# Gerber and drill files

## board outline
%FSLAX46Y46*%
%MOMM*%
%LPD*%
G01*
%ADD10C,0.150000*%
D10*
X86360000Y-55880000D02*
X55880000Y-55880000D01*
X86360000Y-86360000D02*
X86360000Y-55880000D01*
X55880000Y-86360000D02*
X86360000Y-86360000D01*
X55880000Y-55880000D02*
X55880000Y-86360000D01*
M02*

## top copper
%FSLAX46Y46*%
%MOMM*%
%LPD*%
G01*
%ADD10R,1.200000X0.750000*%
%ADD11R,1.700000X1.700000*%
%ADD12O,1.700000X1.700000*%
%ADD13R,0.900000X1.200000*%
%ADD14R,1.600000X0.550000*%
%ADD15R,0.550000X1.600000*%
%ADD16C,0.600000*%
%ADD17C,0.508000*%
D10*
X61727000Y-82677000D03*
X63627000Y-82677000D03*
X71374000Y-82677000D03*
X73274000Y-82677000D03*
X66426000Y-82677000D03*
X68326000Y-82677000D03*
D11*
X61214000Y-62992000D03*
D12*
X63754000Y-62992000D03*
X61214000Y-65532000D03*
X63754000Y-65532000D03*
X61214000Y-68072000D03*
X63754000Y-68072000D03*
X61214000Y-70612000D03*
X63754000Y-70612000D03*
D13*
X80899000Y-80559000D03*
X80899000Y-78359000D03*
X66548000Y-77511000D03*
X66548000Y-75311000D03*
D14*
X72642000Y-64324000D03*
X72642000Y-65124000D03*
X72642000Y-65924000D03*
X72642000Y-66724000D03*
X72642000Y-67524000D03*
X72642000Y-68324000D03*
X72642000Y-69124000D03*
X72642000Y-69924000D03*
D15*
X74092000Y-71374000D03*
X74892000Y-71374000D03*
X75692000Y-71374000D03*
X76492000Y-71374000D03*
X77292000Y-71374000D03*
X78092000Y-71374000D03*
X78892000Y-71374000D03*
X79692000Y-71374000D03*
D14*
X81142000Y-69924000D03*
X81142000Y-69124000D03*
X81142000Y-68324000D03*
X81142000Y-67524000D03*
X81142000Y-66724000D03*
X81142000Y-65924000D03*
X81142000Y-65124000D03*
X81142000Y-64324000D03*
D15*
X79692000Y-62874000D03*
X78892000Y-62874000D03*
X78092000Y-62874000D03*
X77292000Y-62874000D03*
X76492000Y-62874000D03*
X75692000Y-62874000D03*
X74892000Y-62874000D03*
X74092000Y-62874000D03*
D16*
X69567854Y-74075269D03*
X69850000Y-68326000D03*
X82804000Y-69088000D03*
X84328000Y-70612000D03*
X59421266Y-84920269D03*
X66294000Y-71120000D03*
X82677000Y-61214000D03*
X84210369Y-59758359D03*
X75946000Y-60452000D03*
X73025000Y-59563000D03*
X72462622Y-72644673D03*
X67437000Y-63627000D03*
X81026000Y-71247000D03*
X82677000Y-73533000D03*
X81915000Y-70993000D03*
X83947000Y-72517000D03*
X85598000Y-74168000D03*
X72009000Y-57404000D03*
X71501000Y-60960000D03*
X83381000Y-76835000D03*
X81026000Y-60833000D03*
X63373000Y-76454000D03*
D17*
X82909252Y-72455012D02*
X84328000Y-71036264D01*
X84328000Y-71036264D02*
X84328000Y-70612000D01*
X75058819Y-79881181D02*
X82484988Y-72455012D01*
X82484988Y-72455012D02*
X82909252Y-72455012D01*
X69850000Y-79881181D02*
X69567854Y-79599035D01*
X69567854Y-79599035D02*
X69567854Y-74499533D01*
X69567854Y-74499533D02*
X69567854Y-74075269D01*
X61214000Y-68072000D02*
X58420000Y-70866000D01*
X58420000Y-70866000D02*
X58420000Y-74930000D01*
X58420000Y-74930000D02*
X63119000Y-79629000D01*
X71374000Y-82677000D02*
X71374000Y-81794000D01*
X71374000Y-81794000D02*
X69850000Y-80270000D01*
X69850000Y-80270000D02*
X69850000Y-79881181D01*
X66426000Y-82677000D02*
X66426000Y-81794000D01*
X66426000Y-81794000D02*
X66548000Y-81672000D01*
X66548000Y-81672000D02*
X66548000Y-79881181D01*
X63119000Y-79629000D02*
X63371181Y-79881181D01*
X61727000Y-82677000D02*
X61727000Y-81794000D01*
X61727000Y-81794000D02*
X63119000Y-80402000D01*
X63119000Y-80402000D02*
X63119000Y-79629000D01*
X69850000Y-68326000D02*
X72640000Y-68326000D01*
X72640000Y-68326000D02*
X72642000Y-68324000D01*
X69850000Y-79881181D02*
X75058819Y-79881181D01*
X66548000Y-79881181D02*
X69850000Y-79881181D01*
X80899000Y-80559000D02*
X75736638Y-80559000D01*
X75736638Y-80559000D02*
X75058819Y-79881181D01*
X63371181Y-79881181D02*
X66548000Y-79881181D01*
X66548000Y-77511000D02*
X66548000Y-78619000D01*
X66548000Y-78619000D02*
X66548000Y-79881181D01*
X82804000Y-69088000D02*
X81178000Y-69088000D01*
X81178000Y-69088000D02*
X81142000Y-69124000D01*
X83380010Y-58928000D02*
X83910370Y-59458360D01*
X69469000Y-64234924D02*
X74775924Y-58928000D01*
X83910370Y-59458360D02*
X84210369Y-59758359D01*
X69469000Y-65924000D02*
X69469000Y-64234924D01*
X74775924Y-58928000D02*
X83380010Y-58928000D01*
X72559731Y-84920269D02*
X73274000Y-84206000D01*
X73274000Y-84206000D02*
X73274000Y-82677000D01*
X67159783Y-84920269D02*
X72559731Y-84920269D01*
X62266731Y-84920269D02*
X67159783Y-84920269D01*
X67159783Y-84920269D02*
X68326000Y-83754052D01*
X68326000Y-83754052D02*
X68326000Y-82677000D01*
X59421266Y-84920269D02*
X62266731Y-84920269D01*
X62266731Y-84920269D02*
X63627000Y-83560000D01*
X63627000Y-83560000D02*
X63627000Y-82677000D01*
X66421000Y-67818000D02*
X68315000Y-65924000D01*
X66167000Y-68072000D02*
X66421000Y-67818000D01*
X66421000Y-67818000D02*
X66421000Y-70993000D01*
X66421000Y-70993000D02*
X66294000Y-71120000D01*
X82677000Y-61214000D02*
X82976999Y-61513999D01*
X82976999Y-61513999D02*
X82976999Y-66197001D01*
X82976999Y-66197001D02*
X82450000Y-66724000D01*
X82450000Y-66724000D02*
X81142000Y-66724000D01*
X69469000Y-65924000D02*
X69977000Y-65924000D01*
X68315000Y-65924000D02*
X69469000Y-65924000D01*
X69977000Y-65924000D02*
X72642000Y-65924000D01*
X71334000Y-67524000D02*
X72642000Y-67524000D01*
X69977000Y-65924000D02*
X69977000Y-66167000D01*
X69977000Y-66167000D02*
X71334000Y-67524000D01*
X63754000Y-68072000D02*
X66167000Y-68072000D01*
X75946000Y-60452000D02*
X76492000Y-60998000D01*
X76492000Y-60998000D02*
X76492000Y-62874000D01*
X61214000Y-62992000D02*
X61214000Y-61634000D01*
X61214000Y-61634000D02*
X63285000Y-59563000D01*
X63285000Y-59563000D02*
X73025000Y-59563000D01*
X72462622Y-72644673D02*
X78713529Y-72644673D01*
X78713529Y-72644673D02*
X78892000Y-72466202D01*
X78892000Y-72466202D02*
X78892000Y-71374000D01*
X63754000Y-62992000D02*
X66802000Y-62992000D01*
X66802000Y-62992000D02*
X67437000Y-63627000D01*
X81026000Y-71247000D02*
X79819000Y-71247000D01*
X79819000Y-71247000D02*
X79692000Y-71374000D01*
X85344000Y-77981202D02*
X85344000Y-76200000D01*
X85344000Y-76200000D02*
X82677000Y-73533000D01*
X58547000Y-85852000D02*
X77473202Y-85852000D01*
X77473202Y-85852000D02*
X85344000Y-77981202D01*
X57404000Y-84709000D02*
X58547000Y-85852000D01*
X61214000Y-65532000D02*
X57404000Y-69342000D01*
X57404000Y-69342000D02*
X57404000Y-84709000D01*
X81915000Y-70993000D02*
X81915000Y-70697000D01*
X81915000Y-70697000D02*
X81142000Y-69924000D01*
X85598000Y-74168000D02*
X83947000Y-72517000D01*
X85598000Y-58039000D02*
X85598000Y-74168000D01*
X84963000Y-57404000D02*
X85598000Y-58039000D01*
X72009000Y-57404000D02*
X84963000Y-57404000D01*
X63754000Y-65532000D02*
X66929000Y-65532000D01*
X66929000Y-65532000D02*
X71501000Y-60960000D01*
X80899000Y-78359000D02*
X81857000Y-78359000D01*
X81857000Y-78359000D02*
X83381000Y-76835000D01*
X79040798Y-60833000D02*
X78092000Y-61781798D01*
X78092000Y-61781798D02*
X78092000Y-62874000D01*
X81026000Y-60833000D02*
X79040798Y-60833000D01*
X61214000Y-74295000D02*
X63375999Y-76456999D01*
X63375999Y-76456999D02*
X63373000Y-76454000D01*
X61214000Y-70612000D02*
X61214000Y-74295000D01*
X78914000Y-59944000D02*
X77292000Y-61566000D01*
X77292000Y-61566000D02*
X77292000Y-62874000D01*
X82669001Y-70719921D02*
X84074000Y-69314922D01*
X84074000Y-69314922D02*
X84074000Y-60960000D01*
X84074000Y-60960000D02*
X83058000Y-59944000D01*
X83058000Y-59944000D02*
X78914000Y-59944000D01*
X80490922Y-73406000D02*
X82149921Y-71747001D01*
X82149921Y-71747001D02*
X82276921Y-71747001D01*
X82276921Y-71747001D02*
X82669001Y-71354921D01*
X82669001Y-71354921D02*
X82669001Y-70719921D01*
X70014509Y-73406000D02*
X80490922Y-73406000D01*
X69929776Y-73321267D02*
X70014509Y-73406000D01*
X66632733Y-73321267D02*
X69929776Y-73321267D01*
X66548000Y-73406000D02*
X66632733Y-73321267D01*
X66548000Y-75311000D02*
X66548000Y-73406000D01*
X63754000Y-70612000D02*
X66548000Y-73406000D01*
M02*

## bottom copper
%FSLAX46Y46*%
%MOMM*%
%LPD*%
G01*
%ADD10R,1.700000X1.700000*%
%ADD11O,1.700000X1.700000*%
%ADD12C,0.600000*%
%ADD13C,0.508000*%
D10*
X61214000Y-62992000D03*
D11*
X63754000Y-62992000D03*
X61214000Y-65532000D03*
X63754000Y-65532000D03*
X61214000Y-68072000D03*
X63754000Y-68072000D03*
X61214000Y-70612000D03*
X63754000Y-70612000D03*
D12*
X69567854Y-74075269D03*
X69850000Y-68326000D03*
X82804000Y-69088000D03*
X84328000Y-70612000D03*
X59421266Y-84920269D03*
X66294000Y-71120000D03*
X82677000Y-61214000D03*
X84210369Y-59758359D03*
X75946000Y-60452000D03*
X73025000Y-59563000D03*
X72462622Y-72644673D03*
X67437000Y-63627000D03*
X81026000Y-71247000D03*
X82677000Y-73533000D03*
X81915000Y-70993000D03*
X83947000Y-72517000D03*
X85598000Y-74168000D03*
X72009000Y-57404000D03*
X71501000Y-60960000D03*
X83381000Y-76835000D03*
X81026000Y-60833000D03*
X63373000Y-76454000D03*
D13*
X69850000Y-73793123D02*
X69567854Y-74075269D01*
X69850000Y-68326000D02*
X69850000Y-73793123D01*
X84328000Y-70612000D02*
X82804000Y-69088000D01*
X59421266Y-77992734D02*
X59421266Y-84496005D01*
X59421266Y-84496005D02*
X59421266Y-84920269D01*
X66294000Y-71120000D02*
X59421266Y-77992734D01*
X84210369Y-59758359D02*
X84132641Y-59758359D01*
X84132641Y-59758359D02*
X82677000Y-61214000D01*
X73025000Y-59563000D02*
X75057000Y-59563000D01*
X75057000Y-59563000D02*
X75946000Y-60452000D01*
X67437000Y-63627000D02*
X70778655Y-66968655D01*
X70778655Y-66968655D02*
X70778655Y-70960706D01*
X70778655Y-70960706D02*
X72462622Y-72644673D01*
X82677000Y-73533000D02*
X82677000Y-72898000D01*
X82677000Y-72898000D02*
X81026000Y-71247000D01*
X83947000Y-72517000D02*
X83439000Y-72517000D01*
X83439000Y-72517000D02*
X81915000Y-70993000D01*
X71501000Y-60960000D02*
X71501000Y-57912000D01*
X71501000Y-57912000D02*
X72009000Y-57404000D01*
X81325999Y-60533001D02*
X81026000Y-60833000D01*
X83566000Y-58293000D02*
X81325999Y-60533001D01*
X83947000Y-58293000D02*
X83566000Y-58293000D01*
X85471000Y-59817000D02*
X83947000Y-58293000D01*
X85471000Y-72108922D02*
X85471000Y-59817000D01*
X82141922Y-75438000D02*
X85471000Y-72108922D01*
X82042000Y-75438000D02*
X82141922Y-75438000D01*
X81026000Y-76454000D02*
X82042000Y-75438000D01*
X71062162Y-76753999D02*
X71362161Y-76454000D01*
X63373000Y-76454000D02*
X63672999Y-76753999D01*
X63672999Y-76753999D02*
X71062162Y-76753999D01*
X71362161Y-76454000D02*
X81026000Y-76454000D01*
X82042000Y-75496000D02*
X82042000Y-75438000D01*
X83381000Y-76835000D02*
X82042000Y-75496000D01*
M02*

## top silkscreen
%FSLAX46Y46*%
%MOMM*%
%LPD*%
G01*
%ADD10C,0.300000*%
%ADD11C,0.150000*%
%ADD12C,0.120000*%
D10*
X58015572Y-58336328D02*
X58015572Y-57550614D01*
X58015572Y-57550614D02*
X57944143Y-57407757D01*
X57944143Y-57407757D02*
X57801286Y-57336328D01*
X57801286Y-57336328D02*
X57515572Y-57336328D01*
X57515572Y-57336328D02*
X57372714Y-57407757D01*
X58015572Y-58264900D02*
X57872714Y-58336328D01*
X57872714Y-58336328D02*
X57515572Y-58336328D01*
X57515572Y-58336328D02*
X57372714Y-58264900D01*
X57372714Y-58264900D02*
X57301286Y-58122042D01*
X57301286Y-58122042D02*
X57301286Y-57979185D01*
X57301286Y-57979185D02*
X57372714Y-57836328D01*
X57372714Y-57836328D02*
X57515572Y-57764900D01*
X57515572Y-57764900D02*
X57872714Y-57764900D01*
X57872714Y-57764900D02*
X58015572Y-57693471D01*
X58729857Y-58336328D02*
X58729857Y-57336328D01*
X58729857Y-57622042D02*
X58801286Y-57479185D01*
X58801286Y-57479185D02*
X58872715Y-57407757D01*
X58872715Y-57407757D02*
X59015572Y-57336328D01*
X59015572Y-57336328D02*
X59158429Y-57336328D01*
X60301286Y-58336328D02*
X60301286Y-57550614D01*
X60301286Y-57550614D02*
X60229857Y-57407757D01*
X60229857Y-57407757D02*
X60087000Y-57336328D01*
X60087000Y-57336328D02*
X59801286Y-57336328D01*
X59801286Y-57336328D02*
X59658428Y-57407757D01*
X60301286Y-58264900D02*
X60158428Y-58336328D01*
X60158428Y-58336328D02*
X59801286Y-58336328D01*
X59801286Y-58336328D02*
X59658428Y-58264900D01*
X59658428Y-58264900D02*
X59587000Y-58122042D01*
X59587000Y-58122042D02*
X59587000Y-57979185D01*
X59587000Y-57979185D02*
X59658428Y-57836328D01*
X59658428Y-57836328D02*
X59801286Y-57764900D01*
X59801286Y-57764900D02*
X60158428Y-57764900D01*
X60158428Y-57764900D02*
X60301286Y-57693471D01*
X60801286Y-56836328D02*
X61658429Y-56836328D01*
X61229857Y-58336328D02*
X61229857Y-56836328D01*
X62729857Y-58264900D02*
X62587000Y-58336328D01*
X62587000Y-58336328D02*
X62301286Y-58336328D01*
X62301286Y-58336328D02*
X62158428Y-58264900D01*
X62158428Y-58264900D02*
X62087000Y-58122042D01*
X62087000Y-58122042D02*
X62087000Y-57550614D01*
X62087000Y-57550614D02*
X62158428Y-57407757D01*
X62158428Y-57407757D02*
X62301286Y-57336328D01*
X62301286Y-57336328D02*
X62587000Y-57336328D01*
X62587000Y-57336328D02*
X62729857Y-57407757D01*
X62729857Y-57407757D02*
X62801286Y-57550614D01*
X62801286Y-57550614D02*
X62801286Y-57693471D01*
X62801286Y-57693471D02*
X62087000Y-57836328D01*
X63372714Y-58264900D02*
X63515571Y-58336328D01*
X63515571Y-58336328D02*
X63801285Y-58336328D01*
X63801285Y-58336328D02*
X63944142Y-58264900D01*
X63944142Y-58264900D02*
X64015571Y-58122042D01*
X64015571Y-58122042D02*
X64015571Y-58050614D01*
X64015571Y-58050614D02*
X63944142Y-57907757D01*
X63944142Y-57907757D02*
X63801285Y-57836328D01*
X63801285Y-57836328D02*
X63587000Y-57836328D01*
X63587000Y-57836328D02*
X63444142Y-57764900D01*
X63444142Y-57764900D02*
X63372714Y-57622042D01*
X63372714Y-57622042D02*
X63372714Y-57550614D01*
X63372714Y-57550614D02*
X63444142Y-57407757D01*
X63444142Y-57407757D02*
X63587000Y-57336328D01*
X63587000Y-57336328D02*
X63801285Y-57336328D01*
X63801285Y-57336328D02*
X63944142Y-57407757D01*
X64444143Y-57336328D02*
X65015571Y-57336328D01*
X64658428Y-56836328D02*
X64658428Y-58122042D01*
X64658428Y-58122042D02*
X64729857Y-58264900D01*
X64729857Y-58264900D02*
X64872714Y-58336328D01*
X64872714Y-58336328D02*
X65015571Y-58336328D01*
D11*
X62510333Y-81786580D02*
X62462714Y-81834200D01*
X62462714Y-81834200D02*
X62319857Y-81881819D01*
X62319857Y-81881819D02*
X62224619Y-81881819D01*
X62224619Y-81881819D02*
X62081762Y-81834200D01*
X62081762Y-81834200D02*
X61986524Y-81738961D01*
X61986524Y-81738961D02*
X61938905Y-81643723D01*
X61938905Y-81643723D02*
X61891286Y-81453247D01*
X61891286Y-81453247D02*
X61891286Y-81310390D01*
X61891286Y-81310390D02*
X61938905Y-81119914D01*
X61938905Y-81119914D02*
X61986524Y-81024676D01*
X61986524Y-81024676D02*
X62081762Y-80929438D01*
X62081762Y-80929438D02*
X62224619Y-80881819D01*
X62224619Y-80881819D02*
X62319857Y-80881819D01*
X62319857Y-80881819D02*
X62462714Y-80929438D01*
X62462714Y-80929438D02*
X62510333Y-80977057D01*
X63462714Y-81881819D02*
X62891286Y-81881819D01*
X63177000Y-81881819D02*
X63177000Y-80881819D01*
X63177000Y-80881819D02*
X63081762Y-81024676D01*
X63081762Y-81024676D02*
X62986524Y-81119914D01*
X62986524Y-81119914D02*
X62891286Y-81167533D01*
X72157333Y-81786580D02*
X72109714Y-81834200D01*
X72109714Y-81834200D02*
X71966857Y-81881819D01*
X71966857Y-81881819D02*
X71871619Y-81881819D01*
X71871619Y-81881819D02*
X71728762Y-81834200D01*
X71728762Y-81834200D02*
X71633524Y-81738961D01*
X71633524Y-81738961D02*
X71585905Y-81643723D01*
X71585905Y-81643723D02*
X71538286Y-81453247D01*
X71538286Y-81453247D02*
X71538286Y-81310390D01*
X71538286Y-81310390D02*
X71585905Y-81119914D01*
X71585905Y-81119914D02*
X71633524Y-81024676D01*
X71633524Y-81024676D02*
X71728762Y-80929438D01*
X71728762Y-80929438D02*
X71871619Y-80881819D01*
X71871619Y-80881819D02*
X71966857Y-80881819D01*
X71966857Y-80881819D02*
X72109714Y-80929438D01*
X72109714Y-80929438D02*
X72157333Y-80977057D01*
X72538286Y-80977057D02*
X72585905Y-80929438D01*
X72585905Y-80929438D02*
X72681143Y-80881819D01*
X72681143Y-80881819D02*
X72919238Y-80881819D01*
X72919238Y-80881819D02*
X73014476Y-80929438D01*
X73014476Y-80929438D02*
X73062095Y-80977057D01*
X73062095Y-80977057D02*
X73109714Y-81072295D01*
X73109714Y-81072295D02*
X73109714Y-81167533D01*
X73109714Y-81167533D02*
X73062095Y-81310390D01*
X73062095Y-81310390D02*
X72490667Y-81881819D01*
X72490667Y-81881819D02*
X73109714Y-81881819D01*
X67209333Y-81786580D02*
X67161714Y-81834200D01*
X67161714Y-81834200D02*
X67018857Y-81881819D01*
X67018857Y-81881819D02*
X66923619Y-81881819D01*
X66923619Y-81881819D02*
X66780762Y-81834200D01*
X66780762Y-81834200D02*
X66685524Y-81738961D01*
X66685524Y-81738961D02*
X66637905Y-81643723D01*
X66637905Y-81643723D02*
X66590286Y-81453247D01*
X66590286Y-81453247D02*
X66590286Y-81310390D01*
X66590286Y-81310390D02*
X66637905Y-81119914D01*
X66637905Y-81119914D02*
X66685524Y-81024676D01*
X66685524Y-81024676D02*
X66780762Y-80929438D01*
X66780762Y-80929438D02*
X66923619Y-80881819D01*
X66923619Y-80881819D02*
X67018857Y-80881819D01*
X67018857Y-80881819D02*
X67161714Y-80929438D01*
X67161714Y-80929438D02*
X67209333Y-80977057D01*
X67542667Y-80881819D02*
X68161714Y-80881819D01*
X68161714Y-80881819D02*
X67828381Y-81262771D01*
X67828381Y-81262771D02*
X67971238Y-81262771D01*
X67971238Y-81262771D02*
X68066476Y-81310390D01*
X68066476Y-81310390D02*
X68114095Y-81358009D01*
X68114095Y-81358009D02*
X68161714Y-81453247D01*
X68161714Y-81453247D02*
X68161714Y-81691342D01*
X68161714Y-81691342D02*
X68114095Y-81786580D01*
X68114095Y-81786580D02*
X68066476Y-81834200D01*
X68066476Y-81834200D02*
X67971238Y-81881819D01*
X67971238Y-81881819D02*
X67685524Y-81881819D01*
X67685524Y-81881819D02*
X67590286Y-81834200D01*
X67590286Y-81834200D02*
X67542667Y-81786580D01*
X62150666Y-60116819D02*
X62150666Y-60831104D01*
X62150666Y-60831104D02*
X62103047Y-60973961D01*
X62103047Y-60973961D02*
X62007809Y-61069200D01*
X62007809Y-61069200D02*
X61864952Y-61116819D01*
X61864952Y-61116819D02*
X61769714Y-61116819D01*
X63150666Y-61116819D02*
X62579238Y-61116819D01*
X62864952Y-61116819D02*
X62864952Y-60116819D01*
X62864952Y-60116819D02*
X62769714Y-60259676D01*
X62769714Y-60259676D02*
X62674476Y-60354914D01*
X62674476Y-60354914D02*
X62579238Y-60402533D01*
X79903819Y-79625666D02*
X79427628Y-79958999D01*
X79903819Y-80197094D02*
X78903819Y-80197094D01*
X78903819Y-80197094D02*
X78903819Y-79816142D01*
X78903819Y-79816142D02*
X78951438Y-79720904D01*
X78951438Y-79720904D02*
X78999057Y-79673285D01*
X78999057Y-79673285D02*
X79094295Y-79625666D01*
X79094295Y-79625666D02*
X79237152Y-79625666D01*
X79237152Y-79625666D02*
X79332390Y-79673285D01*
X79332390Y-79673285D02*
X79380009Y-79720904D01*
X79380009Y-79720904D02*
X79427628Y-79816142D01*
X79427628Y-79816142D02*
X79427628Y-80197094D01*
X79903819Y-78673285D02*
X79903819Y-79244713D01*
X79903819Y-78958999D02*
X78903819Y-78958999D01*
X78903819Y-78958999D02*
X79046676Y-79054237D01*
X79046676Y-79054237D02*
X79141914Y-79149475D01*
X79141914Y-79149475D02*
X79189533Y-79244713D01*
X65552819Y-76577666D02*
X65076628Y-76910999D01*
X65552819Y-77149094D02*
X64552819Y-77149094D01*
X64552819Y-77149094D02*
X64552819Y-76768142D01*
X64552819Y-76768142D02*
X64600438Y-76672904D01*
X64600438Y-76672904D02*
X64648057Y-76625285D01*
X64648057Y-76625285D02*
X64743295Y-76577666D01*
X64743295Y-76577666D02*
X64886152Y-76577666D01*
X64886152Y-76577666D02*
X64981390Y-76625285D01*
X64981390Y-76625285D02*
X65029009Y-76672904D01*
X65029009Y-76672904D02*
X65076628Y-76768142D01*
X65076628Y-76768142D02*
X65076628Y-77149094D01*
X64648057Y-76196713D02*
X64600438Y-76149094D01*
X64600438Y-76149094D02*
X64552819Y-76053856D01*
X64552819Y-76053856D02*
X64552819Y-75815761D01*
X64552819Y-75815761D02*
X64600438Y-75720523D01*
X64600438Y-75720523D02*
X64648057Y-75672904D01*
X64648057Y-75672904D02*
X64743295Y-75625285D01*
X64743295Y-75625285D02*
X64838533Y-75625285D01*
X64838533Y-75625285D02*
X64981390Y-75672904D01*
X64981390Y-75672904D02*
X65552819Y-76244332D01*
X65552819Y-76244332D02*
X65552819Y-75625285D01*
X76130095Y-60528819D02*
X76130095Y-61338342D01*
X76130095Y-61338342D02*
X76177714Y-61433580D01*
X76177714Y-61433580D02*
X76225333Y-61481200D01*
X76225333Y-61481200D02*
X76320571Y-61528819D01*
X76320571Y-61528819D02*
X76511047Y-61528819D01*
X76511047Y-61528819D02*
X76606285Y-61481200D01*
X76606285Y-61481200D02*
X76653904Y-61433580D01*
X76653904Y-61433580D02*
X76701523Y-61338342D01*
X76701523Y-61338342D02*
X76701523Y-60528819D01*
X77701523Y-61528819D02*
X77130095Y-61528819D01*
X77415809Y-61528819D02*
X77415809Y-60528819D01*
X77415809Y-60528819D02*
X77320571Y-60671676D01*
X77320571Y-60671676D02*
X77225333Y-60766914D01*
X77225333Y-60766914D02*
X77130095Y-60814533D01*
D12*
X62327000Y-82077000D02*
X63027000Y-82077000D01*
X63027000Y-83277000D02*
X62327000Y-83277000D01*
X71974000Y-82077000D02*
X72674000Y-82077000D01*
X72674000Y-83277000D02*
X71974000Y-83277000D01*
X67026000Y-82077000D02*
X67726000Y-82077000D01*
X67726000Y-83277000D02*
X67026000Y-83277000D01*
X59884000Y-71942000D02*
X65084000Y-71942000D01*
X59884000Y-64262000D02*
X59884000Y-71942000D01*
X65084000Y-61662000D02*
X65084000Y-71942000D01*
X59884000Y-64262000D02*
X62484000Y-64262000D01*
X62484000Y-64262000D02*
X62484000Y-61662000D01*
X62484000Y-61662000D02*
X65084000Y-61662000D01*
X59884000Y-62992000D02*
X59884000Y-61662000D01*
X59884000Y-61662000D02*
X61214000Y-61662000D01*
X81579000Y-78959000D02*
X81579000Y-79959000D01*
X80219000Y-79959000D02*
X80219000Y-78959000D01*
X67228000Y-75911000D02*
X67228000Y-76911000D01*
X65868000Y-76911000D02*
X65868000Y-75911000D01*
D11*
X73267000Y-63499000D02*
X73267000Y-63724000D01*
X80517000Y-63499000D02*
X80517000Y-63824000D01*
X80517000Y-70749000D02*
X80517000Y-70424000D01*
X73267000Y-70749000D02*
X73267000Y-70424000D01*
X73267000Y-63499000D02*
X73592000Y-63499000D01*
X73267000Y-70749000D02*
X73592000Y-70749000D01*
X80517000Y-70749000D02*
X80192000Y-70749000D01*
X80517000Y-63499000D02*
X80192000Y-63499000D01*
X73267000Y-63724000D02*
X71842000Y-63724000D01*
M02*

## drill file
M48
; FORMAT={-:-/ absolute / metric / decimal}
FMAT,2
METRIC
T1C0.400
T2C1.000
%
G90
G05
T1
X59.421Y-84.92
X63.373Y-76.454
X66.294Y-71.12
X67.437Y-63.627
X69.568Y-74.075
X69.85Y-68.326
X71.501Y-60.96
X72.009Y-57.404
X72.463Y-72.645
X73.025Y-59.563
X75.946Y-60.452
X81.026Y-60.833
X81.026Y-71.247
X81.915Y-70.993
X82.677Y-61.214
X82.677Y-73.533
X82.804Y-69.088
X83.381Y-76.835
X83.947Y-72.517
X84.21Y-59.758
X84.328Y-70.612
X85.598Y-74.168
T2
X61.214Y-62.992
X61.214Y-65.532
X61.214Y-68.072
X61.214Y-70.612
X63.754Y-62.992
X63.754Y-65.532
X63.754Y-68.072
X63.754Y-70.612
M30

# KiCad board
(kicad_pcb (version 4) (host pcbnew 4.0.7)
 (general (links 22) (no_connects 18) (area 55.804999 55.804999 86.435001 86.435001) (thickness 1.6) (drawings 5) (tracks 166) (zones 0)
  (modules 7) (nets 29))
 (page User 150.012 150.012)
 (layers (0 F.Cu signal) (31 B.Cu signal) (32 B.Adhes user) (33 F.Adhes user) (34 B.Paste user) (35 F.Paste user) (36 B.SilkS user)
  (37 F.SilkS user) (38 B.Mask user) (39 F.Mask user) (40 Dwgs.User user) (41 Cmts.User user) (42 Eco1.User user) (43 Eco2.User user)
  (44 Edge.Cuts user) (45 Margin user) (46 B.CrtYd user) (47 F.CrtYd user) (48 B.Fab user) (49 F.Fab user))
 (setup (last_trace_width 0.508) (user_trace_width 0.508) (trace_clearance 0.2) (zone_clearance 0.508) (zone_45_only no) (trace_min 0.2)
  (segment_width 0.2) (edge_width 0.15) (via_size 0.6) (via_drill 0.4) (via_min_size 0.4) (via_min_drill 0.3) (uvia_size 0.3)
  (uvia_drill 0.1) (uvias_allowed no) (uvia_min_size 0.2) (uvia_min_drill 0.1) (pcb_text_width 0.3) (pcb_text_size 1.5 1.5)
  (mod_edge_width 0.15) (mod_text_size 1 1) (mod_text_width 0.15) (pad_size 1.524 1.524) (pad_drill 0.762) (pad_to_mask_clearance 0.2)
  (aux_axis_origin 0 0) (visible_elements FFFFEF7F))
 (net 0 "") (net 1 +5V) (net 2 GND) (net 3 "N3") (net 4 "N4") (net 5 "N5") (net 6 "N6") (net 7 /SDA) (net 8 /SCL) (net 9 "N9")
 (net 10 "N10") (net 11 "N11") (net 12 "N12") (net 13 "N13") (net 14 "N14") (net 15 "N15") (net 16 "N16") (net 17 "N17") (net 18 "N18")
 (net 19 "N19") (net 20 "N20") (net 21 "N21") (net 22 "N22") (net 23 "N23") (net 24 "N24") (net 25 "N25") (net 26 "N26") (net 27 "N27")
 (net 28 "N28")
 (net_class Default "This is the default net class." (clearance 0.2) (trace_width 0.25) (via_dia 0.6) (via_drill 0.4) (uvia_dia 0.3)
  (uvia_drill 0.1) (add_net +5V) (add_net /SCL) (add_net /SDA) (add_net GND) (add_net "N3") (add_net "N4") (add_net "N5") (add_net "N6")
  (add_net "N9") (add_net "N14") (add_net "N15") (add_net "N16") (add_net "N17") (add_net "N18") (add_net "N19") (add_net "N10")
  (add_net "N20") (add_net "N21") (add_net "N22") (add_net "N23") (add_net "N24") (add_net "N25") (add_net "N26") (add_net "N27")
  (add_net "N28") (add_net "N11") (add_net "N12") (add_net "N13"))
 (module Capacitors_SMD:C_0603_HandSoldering (layer F.Cu) (at 62.677 82.677)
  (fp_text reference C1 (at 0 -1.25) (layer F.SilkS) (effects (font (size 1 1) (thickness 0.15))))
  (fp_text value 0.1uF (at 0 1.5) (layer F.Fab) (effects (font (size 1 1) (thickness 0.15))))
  (fp_line (start -0.35 -0.6) (end 0.35 -0.6) (layer F.SilkS) (width 0.12))
  (fp_line (start 0.35 0.6) (end -0.35 0.6) (layer F.SilkS) (width 0.12))
  (pad 1 smd rect (at -0.95 0) (size 1.2 0.75) (layers F.Cu F.Paste F.Mask) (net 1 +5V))
  (pad 2 smd rect (at 0.95 0) (size 1.2 0.75) (layers F.Cu F.Paste F.Mask) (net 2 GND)))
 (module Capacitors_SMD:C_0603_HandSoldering (layer F.Cu) (at 72.324 82.677)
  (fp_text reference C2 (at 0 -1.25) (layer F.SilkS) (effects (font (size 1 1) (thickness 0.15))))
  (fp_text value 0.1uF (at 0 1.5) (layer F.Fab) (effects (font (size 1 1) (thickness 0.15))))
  (fp_line (start -0.35 -0.6) (end 0.35 -0.6) (layer F.SilkS) (width 0.12))
  (fp_line (start 0.35 0.6) (end -0.35 0.6) (layer F.SilkS) (width 0.12))
  (pad 1 smd rect (at -0.95 0) (size 1.2 0.75) (layers F.Cu F.Paste F.Mask) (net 1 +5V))
  (pad 2 smd rect (at 0.95 0) (size 1.2 0.75) (layers F.Cu F.Paste F.Mask) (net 2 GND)))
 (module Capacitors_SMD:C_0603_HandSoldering (layer F.Cu) (at 67.376 82.677)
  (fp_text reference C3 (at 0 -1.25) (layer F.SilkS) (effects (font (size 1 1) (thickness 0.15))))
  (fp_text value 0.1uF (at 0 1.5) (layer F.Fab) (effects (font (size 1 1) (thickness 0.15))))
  (fp_line (start -0.35 -0.6) (end 0.35 -0.6) (layer F.SilkS) (width 0.12))
  (fp_line (start 0.35 0.6) (end -0.35 0.6) (layer F.SilkS) (width 0.12))
  (pad 1 smd rect (at -0.95 0) (size 1.2 0.75) (layers F.Cu F.Paste F.Mask) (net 1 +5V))
  (pad 2 smd rect (at 0.95 0) (size 1.2 0.75) (layers F.Cu F.Paste F.Mask) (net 2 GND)))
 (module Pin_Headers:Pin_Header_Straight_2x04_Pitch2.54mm (layer F.Cu) (at 61.214 62.992)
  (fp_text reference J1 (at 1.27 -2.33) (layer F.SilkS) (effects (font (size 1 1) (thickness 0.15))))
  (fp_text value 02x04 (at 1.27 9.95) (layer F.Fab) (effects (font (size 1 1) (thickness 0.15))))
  (fp_line (start -1.33 8.95) (end 3.87 8.95) (layer F.SilkS) (width 0.12))
  (fp_line (start -1.33 1.27) (end -1.33 8.95) (layer F.SilkS) (width 0.12))
  (fp_line (start 3.87 -1.33) (end 3.87 8.95) (layer F.SilkS) (width 0.12))
  (fp_line (start -1.33 1.27) (end 1.27 1.27) (layer F.SilkS) (width 0.12))
  (fp_line (start 1.27 1.27) (end 1.27 -1.33) (layer F.SilkS) (width 0.12))
  (fp_line (start 1.27 -1.33) (end 3.87 -1.33) (layer F.SilkS) (width 0.12))
  (fp_line (start -1.33 0) (end -1.33 -1.33) (layer F.SilkS) (width 0.12))
  (fp_line (start -1.33 -1.33) (end 0 -1.33) (layer F.SilkS) (width 0.12))
  (pad 1 thru_hole rect (at 0 0) (size 1.7 1.7) (drill 1) (layers *.Cu *.Mask) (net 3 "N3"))
  (pad 2 thru_hole oval (at 2.54 0) (size 1.7 1.7) (drill 1) (layers *.Cu *.Mask) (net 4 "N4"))
  (pad 3 thru_hole oval (at 0 2.54) (size 1.7 1.7) (drill 1) (layers *.Cu *.Mask) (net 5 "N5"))
  (pad 4 thru_hole oval (at 2.54 2.54) (size 1.7 1.7) (drill 1) (layers *.Cu *.Mask) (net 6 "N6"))
  (pad 5 thru_hole oval (at 0 5.08) (size 1.7 1.7) (drill 1) (layers *.Cu *.Mask) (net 1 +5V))
  (pad 6 thru_hole oval (at 2.54 5.08) (size 1.7 1.7) (drill 1) (layers *.Cu *.Mask) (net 2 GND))
  (pad 7 thru_hole oval (at 0 7.62) (size 1.7 1.7) (drill 1) (layers *.Cu *.Mask) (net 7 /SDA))
  (pad 8 thru_hole oval (at 2.54 7.62) (size 1.7 1.7) (drill 1) (layers *.Cu *.Mask) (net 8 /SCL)))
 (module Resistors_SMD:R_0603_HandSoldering (layer F.Cu) (at 80.899 79.459 90)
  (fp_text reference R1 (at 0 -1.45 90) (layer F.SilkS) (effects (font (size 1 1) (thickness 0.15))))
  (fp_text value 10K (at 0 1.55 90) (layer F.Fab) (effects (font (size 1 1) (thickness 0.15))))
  (fp_line (start 0.5 0.68) (end -0.5 0.68) (layer F.SilkS) (width 0.12))
  (fp_line (start -0.5 -0.68) (end 0.5 -0.68) (layer F.SilkS) (width 0.12))
  (pad 1 smd rect (at -1.1 0 90) (size 1.2 0.9) (layers F.Cu F.Paste F.Mask) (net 1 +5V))
  (pad 2 smd rect (at 1.1 0 90) (size 1.2 0.9) (layers F.Cu F.Paste F.Mask) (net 7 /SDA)))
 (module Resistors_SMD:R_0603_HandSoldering (layer F.Cu) (at 66.548 76.411 90)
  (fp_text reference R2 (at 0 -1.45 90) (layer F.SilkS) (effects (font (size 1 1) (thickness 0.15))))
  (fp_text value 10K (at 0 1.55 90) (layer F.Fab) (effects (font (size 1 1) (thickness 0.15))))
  (fp_line (start 0.5 0.68) (end -0.5 0.68) (layer F.SilkS) (width 0.12))
  (fp_line (start -0.5 -0.68) (end 0.5 -0.68) (layer F.SilkS) (width 0.12))
  (pad 1 smd rect (at -1.1 0 90) (size 1.2 0.9) (layers F.Cu F.Paste F.Mask) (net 1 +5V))
  (pad 2 smd rect (at 1.1 0 90) (size 1.2 0.9) (layers F.Cu F.Paste F.Mask) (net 8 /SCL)))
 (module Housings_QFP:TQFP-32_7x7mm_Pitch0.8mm (layer F.Cu) (at 76.892 67.124)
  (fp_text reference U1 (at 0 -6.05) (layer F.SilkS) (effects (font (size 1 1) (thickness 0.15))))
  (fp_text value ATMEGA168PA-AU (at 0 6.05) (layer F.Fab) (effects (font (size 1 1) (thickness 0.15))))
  (fp_line (start -3.625 -3.625) (end -3.625 -3.4) (layer F.SilkS) (width 0.15))
  (fp_line (start 3.625 -3.625) (end 3.625 -3.3) (layer F.SilkS) (width 0.15))
  (fp_line (start 3.625 3.625) (end 3.625 3.3) (layer F.SilkS) (width 0.15))
  (fp_line (start -3.625 3.625) (end -3.625 3.3) (layer F.SilkS) (width 0.15))
  (fp_line (start -3.625 -3.625) (end -3.3 -3.625) (layer F.SilkS) (width 0.15))
  (fp_line (start -3.625 3.625) (end -3.3 3.625) (layer F.SilkS) (width 0.15))
  (fp_line (start 3.625 3.625) (end 3.3 3.625) (layer F.SilkS) (width 0.15))
  (fp_line (start 3.625 -3.625) (end 3.3 -3.625) (layer F.SilkS) (width 0.15))
  (fp_line (start -3.625 -3.4) (end -5.05 -3.4) (layer F.SilkS) (width 0.15))
  (pad 1 smd rect (at -4.25 -2.8) (size 1.6 0.55) (layers F.Cu F.Paste F.Mask) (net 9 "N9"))
  (pad 2 smd rect (at -4.25 -2) (size 1.6 0.55) (layers F.Cu F.Paste F.Mask) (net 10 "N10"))
  (pad 3 smd rect (at -4.25 -1.2) (size 1.6 0.55) (layers F.Cu F.Paste F.Mask) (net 2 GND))
  (pad 4 smd rect (at -4.25 -0.4) (size 1.6 0.55) (layers F.Cu F.Paste F.Mask) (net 1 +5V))
  (pad 5 smd rect (at -4.25 0.4) (size 1.6 0.55) (layers F.Cu F.Paste F.Mask) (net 2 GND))
  (pad 6 smd rect (at -4.25 1.2) (size 1.6 0.55) (layers F.Cu F.Paste F.Mask) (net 1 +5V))
  (pad 7 smd rect (at -4.25 2) (size 1.6 0.55) (layers F.Cu F.Paste F.Mask) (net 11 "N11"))
  (pad 8 smd rect (at -4.25 2.8) (size 1.6 0.55) (layers F.Cu F.Paste F.Mask) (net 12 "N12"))
  (pad 9 smd rect (at -2.8 4.25 90) (size 1.6 0.55) (layers F.Cu F.Paste F.Mask) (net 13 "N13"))
  (pad 10 smd rect (at -2 4.25 90) (size 1.6 0.55) (layers F.Cu F.Paste F.Mask) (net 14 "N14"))
  (pad 11 smd rect (at -1.2 4.25 90) (size 1.6 0.55) (layers F.Cu F.Paste F.Mask) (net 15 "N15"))
  (pad 12 smd rect (at -0.4 4.25 90) (size 1.6 0.55) (layers F.Cu F.Paste F.Mask) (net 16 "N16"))
  (pad 13 smd rect (at 0.4 4.25 90) (size 1.6 0.55) (layers F.Cu F.Paste F.Mask) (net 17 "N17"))
  (pad 14 smd rect (at 1.2 4.25 90) (size 1.6 0.55) (layers F.Cu F.Paste F.Mask) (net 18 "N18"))
  (pad 15 smd rect (at 2 4.25 90) (size 1.6 0.55) (layers F.Cu F.Paste F.Mask) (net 4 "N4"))
  (pad 16 smd rect (at 2.8 4.25 90) (size 1.6 0.55) (layers F.Cu F.Paste F.Mask) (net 5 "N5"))
  (pad 17 smd rect (at 4.25 2.8) (size 1.6 0.55) (layers F.Cu F.Paste F.Mask) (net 6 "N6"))
  (pad 18 smd rect (at 4.25 2) (size 1.6 0.55) (layers F.Cu F.Paste F.Mask) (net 1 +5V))
  (pad 19 smd rect (at 4.25 1.2) (size 1.6 0.55) (layers F.Cu F.Paste F.Mask) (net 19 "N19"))
  (pad 20 smd rect (at 4.25 0.4) (size 1.6 0.55) (layers F.Cu F.Paste F.Mask) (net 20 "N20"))
  (pad 21 smd rect (at 4.25 -0.4) (size 1.6 0.55) (layers F.Cu F.Paste F.Mask) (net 2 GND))
  (pad 22 smd rect (at 4.25 -1.2) (size 1.6 0.55) (layers F.Cu F.Paste F.Mask) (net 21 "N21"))
  (pad 23 smd rect (at 4.25 -2) (size 1.6 0.55) (layers F.Cu F.Paste F.Mask) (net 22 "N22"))
  (pad 24 smd rect (at 4.25 -2.8) (size 1.6 0.55) (layers F.Cu F.Paste F.Mask) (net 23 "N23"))
  (pad 25 smd rect (at 2.8 -4.25 90) (size 1.6 0.55) (layers F.Cu F.Paste F.Mask) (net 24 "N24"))
  (pad 26 smd rect (at 2 -4.25 90) (size 1.6 0.55) (layers F.Cu F.Paste F.Mask) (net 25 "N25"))
  (pad 27 smd rect (at 1.2 -4.25 90) (size 1.6 0.55) (layers F.Cu F.Paste F.Mask) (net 7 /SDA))
  (pad 28 smd rect (at 0.4 -4.25 90) (size 1.6 0.55) (layers F.Cu F.Paste F.Mask) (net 8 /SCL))
  (pad 29 smd rect (at -0.4 -4.25 90) (size 1.6 0.55) (layers F.Cu F.Paste F.Mask) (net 3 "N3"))
  (pad 30 smd rect (at -1.2 -4.25 90) (size 1.6 0.55) (layers F.Cu F.Paste F.Mask) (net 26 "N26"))
  (pad 31 smd rect (at -2 -4.25 90) (size 1.6 0.55) (layers F.Cu F.Paste F.Mask) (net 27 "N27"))
  (pad 32 smd rect (at -2.8 -4.25 90) (size 1.6 0.55) (layers F.Cu F.Paste F.Mask) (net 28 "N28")))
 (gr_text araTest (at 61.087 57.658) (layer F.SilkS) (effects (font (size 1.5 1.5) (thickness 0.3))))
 (gr_line (start 86.36 55.88) (end 55.88 55.88) (layer Edge.Cuts) (width 0.15))
 (gr_line (start 86.36 86.36) (end 86.36 55.88) (layer Edge.Cuts) (width 0.15))
 (gr_line (start 55.88 86.36) (end 86.36 86.36) (layer Edge.Cuts) (width 0.15))
 (gr_line (start 55.88 55.88) (end 55.88 86.36) (layer Edge.Cuts) (width 0.15))
 (segment (start 82.909252 72.455012) (end 84.328 71.036264) (width 0.508) (layer F.Cu) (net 1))
 (segment (start 84.328 71.036264) (end 84.328 70.612) (width 0.508) (layer F.Cu) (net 1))
 (segment (start 75.058819 79.881181) (end 82.484988 72.455012) (width 0.508) (layer F.Cu) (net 1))
 (segment (start 82.484988 72.455012) (end 82.909252 72.455012) (width 0.508) (layer F.Cu) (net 1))
 (segment (start 69.85 79.881181) (end 69.567854 79.599035) (width 0.508) (layer F.Cu) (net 1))
 (via (at 69.567854 74.075269) (size 0.6) (drill 0.4) (layers F.Cu B.Cu) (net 1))
 (segment (start 69.567854 79.599035) (end 69.567854 74.499533) (width 0.508) (layer F.Cu) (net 1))
 (segment (start 69.567854 74.499533) (end 69.567854 74.075269) (width 0.508) (layer F.Cu) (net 1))
 (segment (start 69.85 73.793123) (end 69.567854 74.075269) (width 0.508) (layer B.Cu) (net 1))
 (segment (start 69.85 68.326) (end 69.85 73.793123) (width 0.508) (layer B.Cu) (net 1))
 (segment (start 61.214 68.072) (end 58.42 70.866) (width 0.508) (layer F.Cu) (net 1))
 (segment (start 58.42 70.866) (end 58.42 74.93) (width 0.508) (layer F.Cu) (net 1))
 (segment (start 58.42 74.93) (end 63.119 79.629) (width 0.508) (layer F.Cu) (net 1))
 (segment (start 71.374 82.677) (end 71.374 81.794) (width 0.508) (layer F.Cu) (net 1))
 (segment (start 71.374 81.794) (end 69.85 80.27) (width 0.508) (layer F.Cu) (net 1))
 (segment (start 69.85 80.27) (end 69.85 79.881181) (width 0.508) (layer F.Cu) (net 1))
 (segment (start 66.426 82.677) (end 66.426 81.794) (width 0.508) (layer F.Cu) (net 1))
 (segment (start 66.426 81.794) (end 66.548 81.672) (width 0.508) (layer F.Cu) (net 1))
 (segment (start 66.548 81.672) (end 66.548 79.881181) (width 0.508) (layer F.Cu) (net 1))
 (segment (start 63.119 79.629) (end 63.371181 79.881181) (width 0.508) (layer F.Cu) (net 1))
 (segment (start 61.727 82.677) (end 61.727 81.794) (width 0.508) (layer F.Cu) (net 1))
 (segment (start 61.727 81.794) (end 63.119 80.402) (width 0.508) (layer F.Cu) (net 1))
 (segment (start 63.119 80.402) (end 63.119 79.629) (width 0.508) (layer F.Cu) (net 1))
 (segment (start 69.85 68.326) (end 72.64 68.326) (width 0.508) (layer F.Cu) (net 1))
 (segment (start 72.64 68.326) (end 72.642 68.324) (width 0.508) (layer F.Cu) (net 1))
 (via (at 69.85 68.326) (size 0.6) (drill 0.4) (layers F.Cu B.Cu) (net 1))
 (segment (start 69.85 79.881181) (end 75.058819 79.881181) (width 0.508) (layer F.Cu) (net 1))
 (segment (start 66.548 79.881181) (end 69.85 79.881181) (width 0.508) (layer F.Cu) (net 1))
 (segment (start 80.899 80.559) (end 75.736638 80.559) (width 0.508) (layer F.Cu) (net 1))
 (segment (start 75.736638 80.559) (end 75.058819 79.881181) (width 0.508) (layer F.Cu) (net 1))
 (segment (start 63.371181 79.881181) (end 66.548 79.881181) (width 0.508) (layer F.Cu) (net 1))
 (segment (start 66.548 77.511) (end 66.548 78.619) (width 0.508) (layer F.Cu) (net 1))
 (segment (start 66.548 78.619) (end 66.548 79.881181) (width 0.508) (layer F.Cu) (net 1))
 (segment (start 82.804 69.088) (end 81.178 69.088) (width 0.508) (layer F.Cu) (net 1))
 (segment (start 81.178 69.088) (end 81.142 69.124) (width 0.508) (layer F.Cu) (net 1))
 (segment (start 84.328 70.612) (end 82.804 69.088) (width 0.508) (layer B.Cu) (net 1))
 (via (at 82.804 69.088) (size 0.6) (drill 0.4) (layers F.Cu B.Cu) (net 1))
 (via (at 84.328 70.612) (size 0.6) (drill 0.4) (layers F.Cu B.Cu) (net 1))
 (segment (start 83.38001 58.928) (end 83.91037 59.45836) (width 0.508) (layer F.Cu) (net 2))
 (segment (start 69.469 64.234924) (end 74.775924 58.928) (width 0.508) (layer F.Cu) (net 2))
 (segment (start 83.91037 59.45836) (end 84.210369 59.758359) (width 0.508) (layer F.Cu) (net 2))
 (segment (start 69.469 65.924) (end 69.469 64.234924) (width 0.508) (layer F.Cu) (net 2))
 (segment (start 74.775924 58.928) (end 83.38001 58.928) (width 0.508) (layer F.Cu) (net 2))
 (segment (start 72.559731 84.920269) (end 73.274 84.206) (width 0.508) (layer F.Cu) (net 2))
 (segment (start 73.274 84.206) (end 73.274 82.677) (width 0.508) (layer F.Cu) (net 2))
 (segment (start 67.159783 84.920269) (end 72.559731 84.920269) (width 0.508) (layer F.Cu) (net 2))
 (segment (start 62.266731 84.920269) (end 67.159783 84.920269) (width 0.508) (layer F.Cu) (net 2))
 (segment (start 67.159783 84.920269) (end 68.326 83.754052) (width 0.508) (layer F.Cu) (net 2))
 (segment (start 68.326 83.754052) (end 68.326 82.677) (width 0.508) (layer F.Cu) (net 2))
 (segment (start 59.421266 84.920269) (end 62.266731 84.920269) (width 0.508) (layer F.Cu) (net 2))
 (segment (start 62.266731 84.920269) (end 63.627 83.56) (width 0.508) (layer F.Cu) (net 2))
 (segment (start 63.627 83.56) (end 63.627 82.677) (width 0.508) (layer F.Cu) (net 2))
 (segment (start 59.421266 77.992734) (end 59.421266 84.496005) (width 0.508) (layer B.Cu) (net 2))
 (segment (start 59.421266 84.496005) (end 59.421266 84.920269) (width 0.508) (layer B.Cu) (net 2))
 (segment (start 66.294 71.12) (end 59.421266 77.992734) (width 0.508) (layer B.Cu) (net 2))
 (via (at 59.421266 84.920269) (size 0.6) (drill 0.4) (layers F.Cu B.Cu) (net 2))
 (segment (start 66.421 67.818) (end 68.315 65.924) (width 0.508) (layer F.Cu) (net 2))
 (segment (start 66.167 68.072) (end 66.421 67.818) (width 0.508) (layer F.Cu) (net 2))
 (segment (start 66.421 67.818) (end 66.421 70.993) (width 0.508) (layer F.Cu) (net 2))
 (segment (start 66.421 70.993) (end 66.294 71.12) (width 0.508) (layer F.Cu) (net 2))
 (via (at 66.294 71.12) (size 0.6) (drill 0.4) (layers F.Cu B.Cu) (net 2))
 (segment (start 82.677 61.214) (end 82.976999 61.513999) (width 0.508) (layer F.Cu) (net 2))
 (segment (start 82.976999 61.513999) (end 82.976999 66.197001) (width 0.508) (layer F.Cu) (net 2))
 (segment (start 82.976999 66.197001) (end 82.45 66.724) (width 0.508) (layer F.Cu) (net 2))
 (segment (start 82.45 66.724) (end 81.142 66.724) (width 0.508) (layer F.Cu) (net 2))
 (segment (start 84.210369 59.758359) (end 84.132641 59.758359) (width 0.508) (layer B.Cu) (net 2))
 (segment (start 84.132641 59.758359) (end 82.677 61.214) (width 0.508) (layer B.Cu) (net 2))
 (via (at 82.677 61.214) (size 0.6) (drill 0.4) (layers F.Cu B.Cu) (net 2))
 (via (at 84.210369 59.758359) (size 0.6) (drill 0.4) (layers F.Cu B.Cu) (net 2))
 (segment (start 69.469 65.924) (end 69.977 65.924) (width 0.508) (layer F.Cu) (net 2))
 (segment (start 68.315 65.924) (end 69.469 65.924) (width 0.508) (layer F.Cu) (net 2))
 (segment (start 69.977 65.924) (end 72.642 65.924) (width 0.508) (layer F.Cu) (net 2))
 (segment (start 71.334 67.524) (end 72.642 67.524) (width 0.508) (layer F.Cu) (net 2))
 (segment (start 69.977 65.924) (end 69.977 66.167) (width 0.508) (layer F.Cu) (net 2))
 (segment (start 69.977 66.167) (end 71.334 67.524) (width 0.508) (layer F.Cu) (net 2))
 (segment (start 63.754 68.072) (end 66.167 68.072) (width 0.508) (layer F.Cu) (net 2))
 (segment (start 75.946 60.452) (end 76.492 60.998) (width 0.508) (layer F.Cu) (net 3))
 (segment (start 76.492 60.998) (end 76.492 62.874) (width 0.508) (layer F.Cu) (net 3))
 (segment (start 73.025 59.563) (end 75.057 59.563) (width 0.508) (layer B.Cu) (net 3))
 (segment (start 75.057 59.563) (end 75.946 60.452) (width 0.508) (layer B.Cu) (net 3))
 (via (at 75.946 60.452) (size 0.6) (drill 0.4) (layers F.Cu B.Cu) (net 3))
 (via (at 73.025 59.563) (size 0.6) (drill 0.4) (layers F.Cu B.Cu) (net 3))
 (segment (start 61.214 62.992) (end 61.214 61.634) (width 0.508) (layer F.Cu) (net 3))
 (segment (start 61.214 61.634) (end 63.285 59.563) (width 0.508) (layer F.Cu) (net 3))
 (segment (start 63.285 59.563) (end 73.025 59.563) (width 0.508) (layer F.Cu) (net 3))
 (segment (start 72.462622 72.644673) (end 78.713529 72.644673) (width 0.508) (layer F.Cu) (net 4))
 (segment (start 78.713529 72.644673) (end 78.892 72.466202) (width 0.508) (layer F.Cu) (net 4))
 (segment (start 78.892 72.466202) (end 78.892 71.374) (width 0.508) (layer F.Cu) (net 4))
 (via (at 72.462622 72.644673) (size 0.6) (drill 0.4) (layers F.Cu B.Cu) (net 4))
 (segment (start 67.437 63.627) (end 70.778655 66.968655) (width 0.508) (layer B.Cu) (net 4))
 (segment (start 70.778655 66.968655) (end 70.778655 70.960706) (width 0.508) (layer B.Cu) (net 4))
 (segment (start 70.778655 70.960706) (end 72.462622 72.644673) (width 0.508) (layer B.Cu) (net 4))
 (segment (start 63.754 62.992) (end 66.802 62.992) (width 0.508) (layer F.Cu) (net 4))
 (segment (start 66.802 62.992) (end 67.437 63.627) (width 0.508) (layer F.Cu) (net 4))
 (via (at 67.437 63.627) (size 0.6) (drill 0.4) (layers F.Cu B.Cu) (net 4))
 (segment (start 81.026 71.247) (end 79.819 71.247) (width 0.508) (layer F.Cu) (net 5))
 (segment (start 79.819 71.247) (end 79.692 71.374) (width 0.508) (layer F.Cu) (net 5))
 (segment (start 82.677 73.533) (end 82.677 72.898) (width 0.508) (layer B.Cu) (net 5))
 (segment (start 82.677 72.898) (end 81.026 71.247) (width 0.508) (layer B.Cu) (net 5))
 (via (at 81.026 71.247) (size 0.6) (drill 0.4) (layers F.Cu B.Cu) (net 5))
 (segment (start 85.344 77.981202) (end 85.344 76.2) (width 0.508) (layer F.Cu) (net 5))
 (segment (start 85.344 76.2) (end 82.677 73.533) (width 0.508) (layer F.Cu) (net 5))
 (via (at 82.677 73.533) (size 0.6) (drill 0.4) (layers F.Cu B.Cu) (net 5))
 (segment (start 58.547 85.852) (end 77.473202 85.852) (width 0.508) (layer F.Cu) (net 5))
 (segment (start 77.473202 85.852) (end 85.344 77.981202) (width 0.508) (layer F.Cu) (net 5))
 (segment (start 57.404 84.709) (end 58.547 85.852) (width 0.508) (layer F.Cu) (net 5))
 (segment (start 61.214 65.532) (end 57.404 69.342) (width 0.508) (layer F.Cu) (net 5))
 (segment (start 57.404 69.342) (end 57.404 84.709) (width 0.508) (layer F.Cu) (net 5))
 (segment (start 81.915 70.993) (end 81.915 70.697) (width 0.508) (layer F.Cu) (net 6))
 (segment (start 81.915 70.697) (end 81.142 69.924) (width 0.508) (layer F.Cu) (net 6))
 (via (at 81.915 70.993) (size 0.6) (drill 0.4) (layers F.Cu B.Cu) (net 6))
 (segment (start 83.947 72.517) (end 83.439 72.517) (width 0.508) (layer B.Cu) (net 6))
 (segment (start 83.439 72.517) (end 81.915 70.993) (width 0.508) (layer B.Cu) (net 6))
 (segment (start 85.598 74.168) (end 83.947 72.517) (width 0.508) (layer F.Cu) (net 6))
 (via (at 83.947 72.517) (size 0.6) (drill 0.4) (layers F.Cu B.Cu) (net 6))
 (segment (start 85.598 58.039) (end 85.598 74.168) (width 0.508) (layer F.Cu) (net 6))
 (via (at 85.598 74.168) (size 0.6) (drill 0.4) (layers F.Cu B.Cu) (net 6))
 (segment (start 84.963 57.404) (end 85.598 58.039) (width 0.508) (layer F.Cu) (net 6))
 (segment (start 72.009 57.404) (end 84.963 57.404) (width 0.508) (layer F.Cu) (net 6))
 (segment (start 71.501 60.96) (end 71.501 57.912) (width 0.508) (layer B.Cu) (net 6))
 (segment (start 71.501 57.912) (end 72.009 57.404) (width 0.508) (layer B.Cu) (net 6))
 (via (at 72.009 57.404) (size 0.6) (drill 0.4) (layers F.Cu B.Cu) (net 6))
 (segment (start 63.754 65.532) (end 66.929 65.532) (width 0.508) (layer F.Cu) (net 6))
 (segment (start 66.929 65.532) (end 71.501 60.96) (width 0.508) (layer F.Cu) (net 6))
 (via (at 71.501 60.96) (size 0.6) (drill 0.4) (layers F.Cu B.Cu) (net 6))
 (segment (start 81.325999 60.533001) (end 81.026 60.833) (width 0.508) (layer B.Cu) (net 7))
 (segment (start 83.566 58.293) (end 81.325999 60.533001) (width 0.508) (layer B.Cu) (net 7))
 (segment (start 83.947 58.293) (end 83.566 58.293) (width 0.508) (layer B.Cu) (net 7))
 (segment (start 85.471 59.817) (end 83.947 58.293) (width 0.508) (layer B.Cu) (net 7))
 (segment (start 85.471 72.108922) (end 85.471 59.817) (width 0.508) (layer B.Cu) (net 7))
 (segment (start 82.141922 75.438) (end 85.471 72.108922) (width 0.508) (layer B.Cu) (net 7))
 (segment (start 82.042 75.438) (end 82.141922 75.438) (width 0.508) (layer B.Cu) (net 7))
 (segment (start 81.026 76.454) (end 82.042 75.438) (width 0.508) (layer B.Cu) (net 7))
 (segment (start 71.062162 76.753999) (end 71.362161 76.454) (width 0.508) (layer B.Cu) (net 7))
 (segment (start 63.373 76.454) (end 63.672999 76.753999) (width 0.508) (layer B.Cu) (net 7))
 (segment (start 63.672999 76.753999) (end 71.062162 76.753999) (width 0.508) (layer B.Cu) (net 7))
 (segment (start 71.362161 76.454) (end 81.026 76.454) (width 0.508) (layer B.Cu) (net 7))
 (segment (start 82.042 75.496) (end 82.042 75.438) (width 0.508) (layer B.Cu) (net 7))
 (segment (start 83.381 76.835) (end 82.042 75.496) (width 0.508) (layer B.Cu) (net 7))
 (via (at 83.381 76.835) (size 0.6) (drill 0.4) (layers F.Cu B.Cu) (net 7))
 (segment (start 80.899 78.359) (end 81.857 78.359) (width 0.508) (layer F.Cu) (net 7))
 (segment (start 81.857 78.359) (end 83.381 76.835) (width 0.508) (layer F.Cu) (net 7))
 (segment (start 79.040798 60.833) (end 78.092 61.781798) (width 0.508) (layer F.Cu) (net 7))
 (segment (start 78.092 61.781798) (end 78.092 62.874) (width 0.508) (layer F.Cu) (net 7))
 (segment (start 81.026 60.833) (end 79.040798 60.833) (width 0.508) (layer F.Cu) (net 7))
 (via (at 81.026 60.833) (size 0.6) (drill 0.4) (layers F.Cu B.Cu) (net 7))
 (segment (start 61.214 74.295) (end 63.375999 76.456999) (width 0.508) (layer F.Cu) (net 7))
 (segment (start 63.375999 76.456999) (end 63.373 76.454) (width 0.508) (layer F.Cu) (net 7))
 (via (at 63.373 76.454) (size 0.6) (drill 0.4) (layers F.Cu B.Cu) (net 7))
 (segment (start 61.214 70.612) (end 61.214 74.295) (width 0.508) (layer F.Cu) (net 7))
 (segment (start 78.914 59.944) (end 77.292 61.566) (width 0.508) (layer F.Cu) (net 8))
 (segment (start 77.292 61.566) (end 77.292 62.874) (width 0.508) (layer F.Cu) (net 8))
 (segment (start 82.669001 70.719921) (end 84.074 69.314922) (width 0.508) (layer F.Cu) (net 8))
 (segment (start 84.074 69.314922) (end 84.074 60.96) (width 0.508) (layer F.Cu) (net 8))
 (segment (start 84.074 60.96) (end 83.058 59.944) (width 0.508) (layer F.Cu) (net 8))
 (segment (start 83.058 59.944) (end 78.914 59.944) (width 0.508) (layer F.Cu) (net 8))
 (segment (start 80.490922 73.406) (end 82.149921 71.747001) (width 0.508) (layer F.Cu) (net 8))
 (segment (start 82.149921 71.747001) (end 82.276921 71.747001) (width 0.508) (layer F.Cu) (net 8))
 (segment (start 82.276921 71.747001) (end 82.669001 71.354921) (width 0.508) (layer F.Cu) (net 8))
 (segment (start 82.669001 71.354921) (end 82.669001 70.719921) (width 0.508) (layer F.Cu) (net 8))
 (segment (start 70.014509 73.406) (end 80.490922 73.406) (width 0.508) (layer F.Cu) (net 8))
 (segment (start 69.929776 73.321267) (end 70.014509 73.406) (width 0.508) (layer F.Cu) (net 8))
 (segment (start 66.632733 73.321267) (end 69.929776 73.321267) (width 0.508) (layer F.Cu) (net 8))
 (segment (start 66.548 73.406) (end 66.632733 73.321267) (width 0.508) (layer F.Cu) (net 8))
 (segment (start 66.548 75.311) (end 66.548 73.406) (width 0.508) (layer F.Cu) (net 8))
 (segment (start 63.754 70.612) (end 66.548 73.406) (width 0.508) (layer F.Cu) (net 8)))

